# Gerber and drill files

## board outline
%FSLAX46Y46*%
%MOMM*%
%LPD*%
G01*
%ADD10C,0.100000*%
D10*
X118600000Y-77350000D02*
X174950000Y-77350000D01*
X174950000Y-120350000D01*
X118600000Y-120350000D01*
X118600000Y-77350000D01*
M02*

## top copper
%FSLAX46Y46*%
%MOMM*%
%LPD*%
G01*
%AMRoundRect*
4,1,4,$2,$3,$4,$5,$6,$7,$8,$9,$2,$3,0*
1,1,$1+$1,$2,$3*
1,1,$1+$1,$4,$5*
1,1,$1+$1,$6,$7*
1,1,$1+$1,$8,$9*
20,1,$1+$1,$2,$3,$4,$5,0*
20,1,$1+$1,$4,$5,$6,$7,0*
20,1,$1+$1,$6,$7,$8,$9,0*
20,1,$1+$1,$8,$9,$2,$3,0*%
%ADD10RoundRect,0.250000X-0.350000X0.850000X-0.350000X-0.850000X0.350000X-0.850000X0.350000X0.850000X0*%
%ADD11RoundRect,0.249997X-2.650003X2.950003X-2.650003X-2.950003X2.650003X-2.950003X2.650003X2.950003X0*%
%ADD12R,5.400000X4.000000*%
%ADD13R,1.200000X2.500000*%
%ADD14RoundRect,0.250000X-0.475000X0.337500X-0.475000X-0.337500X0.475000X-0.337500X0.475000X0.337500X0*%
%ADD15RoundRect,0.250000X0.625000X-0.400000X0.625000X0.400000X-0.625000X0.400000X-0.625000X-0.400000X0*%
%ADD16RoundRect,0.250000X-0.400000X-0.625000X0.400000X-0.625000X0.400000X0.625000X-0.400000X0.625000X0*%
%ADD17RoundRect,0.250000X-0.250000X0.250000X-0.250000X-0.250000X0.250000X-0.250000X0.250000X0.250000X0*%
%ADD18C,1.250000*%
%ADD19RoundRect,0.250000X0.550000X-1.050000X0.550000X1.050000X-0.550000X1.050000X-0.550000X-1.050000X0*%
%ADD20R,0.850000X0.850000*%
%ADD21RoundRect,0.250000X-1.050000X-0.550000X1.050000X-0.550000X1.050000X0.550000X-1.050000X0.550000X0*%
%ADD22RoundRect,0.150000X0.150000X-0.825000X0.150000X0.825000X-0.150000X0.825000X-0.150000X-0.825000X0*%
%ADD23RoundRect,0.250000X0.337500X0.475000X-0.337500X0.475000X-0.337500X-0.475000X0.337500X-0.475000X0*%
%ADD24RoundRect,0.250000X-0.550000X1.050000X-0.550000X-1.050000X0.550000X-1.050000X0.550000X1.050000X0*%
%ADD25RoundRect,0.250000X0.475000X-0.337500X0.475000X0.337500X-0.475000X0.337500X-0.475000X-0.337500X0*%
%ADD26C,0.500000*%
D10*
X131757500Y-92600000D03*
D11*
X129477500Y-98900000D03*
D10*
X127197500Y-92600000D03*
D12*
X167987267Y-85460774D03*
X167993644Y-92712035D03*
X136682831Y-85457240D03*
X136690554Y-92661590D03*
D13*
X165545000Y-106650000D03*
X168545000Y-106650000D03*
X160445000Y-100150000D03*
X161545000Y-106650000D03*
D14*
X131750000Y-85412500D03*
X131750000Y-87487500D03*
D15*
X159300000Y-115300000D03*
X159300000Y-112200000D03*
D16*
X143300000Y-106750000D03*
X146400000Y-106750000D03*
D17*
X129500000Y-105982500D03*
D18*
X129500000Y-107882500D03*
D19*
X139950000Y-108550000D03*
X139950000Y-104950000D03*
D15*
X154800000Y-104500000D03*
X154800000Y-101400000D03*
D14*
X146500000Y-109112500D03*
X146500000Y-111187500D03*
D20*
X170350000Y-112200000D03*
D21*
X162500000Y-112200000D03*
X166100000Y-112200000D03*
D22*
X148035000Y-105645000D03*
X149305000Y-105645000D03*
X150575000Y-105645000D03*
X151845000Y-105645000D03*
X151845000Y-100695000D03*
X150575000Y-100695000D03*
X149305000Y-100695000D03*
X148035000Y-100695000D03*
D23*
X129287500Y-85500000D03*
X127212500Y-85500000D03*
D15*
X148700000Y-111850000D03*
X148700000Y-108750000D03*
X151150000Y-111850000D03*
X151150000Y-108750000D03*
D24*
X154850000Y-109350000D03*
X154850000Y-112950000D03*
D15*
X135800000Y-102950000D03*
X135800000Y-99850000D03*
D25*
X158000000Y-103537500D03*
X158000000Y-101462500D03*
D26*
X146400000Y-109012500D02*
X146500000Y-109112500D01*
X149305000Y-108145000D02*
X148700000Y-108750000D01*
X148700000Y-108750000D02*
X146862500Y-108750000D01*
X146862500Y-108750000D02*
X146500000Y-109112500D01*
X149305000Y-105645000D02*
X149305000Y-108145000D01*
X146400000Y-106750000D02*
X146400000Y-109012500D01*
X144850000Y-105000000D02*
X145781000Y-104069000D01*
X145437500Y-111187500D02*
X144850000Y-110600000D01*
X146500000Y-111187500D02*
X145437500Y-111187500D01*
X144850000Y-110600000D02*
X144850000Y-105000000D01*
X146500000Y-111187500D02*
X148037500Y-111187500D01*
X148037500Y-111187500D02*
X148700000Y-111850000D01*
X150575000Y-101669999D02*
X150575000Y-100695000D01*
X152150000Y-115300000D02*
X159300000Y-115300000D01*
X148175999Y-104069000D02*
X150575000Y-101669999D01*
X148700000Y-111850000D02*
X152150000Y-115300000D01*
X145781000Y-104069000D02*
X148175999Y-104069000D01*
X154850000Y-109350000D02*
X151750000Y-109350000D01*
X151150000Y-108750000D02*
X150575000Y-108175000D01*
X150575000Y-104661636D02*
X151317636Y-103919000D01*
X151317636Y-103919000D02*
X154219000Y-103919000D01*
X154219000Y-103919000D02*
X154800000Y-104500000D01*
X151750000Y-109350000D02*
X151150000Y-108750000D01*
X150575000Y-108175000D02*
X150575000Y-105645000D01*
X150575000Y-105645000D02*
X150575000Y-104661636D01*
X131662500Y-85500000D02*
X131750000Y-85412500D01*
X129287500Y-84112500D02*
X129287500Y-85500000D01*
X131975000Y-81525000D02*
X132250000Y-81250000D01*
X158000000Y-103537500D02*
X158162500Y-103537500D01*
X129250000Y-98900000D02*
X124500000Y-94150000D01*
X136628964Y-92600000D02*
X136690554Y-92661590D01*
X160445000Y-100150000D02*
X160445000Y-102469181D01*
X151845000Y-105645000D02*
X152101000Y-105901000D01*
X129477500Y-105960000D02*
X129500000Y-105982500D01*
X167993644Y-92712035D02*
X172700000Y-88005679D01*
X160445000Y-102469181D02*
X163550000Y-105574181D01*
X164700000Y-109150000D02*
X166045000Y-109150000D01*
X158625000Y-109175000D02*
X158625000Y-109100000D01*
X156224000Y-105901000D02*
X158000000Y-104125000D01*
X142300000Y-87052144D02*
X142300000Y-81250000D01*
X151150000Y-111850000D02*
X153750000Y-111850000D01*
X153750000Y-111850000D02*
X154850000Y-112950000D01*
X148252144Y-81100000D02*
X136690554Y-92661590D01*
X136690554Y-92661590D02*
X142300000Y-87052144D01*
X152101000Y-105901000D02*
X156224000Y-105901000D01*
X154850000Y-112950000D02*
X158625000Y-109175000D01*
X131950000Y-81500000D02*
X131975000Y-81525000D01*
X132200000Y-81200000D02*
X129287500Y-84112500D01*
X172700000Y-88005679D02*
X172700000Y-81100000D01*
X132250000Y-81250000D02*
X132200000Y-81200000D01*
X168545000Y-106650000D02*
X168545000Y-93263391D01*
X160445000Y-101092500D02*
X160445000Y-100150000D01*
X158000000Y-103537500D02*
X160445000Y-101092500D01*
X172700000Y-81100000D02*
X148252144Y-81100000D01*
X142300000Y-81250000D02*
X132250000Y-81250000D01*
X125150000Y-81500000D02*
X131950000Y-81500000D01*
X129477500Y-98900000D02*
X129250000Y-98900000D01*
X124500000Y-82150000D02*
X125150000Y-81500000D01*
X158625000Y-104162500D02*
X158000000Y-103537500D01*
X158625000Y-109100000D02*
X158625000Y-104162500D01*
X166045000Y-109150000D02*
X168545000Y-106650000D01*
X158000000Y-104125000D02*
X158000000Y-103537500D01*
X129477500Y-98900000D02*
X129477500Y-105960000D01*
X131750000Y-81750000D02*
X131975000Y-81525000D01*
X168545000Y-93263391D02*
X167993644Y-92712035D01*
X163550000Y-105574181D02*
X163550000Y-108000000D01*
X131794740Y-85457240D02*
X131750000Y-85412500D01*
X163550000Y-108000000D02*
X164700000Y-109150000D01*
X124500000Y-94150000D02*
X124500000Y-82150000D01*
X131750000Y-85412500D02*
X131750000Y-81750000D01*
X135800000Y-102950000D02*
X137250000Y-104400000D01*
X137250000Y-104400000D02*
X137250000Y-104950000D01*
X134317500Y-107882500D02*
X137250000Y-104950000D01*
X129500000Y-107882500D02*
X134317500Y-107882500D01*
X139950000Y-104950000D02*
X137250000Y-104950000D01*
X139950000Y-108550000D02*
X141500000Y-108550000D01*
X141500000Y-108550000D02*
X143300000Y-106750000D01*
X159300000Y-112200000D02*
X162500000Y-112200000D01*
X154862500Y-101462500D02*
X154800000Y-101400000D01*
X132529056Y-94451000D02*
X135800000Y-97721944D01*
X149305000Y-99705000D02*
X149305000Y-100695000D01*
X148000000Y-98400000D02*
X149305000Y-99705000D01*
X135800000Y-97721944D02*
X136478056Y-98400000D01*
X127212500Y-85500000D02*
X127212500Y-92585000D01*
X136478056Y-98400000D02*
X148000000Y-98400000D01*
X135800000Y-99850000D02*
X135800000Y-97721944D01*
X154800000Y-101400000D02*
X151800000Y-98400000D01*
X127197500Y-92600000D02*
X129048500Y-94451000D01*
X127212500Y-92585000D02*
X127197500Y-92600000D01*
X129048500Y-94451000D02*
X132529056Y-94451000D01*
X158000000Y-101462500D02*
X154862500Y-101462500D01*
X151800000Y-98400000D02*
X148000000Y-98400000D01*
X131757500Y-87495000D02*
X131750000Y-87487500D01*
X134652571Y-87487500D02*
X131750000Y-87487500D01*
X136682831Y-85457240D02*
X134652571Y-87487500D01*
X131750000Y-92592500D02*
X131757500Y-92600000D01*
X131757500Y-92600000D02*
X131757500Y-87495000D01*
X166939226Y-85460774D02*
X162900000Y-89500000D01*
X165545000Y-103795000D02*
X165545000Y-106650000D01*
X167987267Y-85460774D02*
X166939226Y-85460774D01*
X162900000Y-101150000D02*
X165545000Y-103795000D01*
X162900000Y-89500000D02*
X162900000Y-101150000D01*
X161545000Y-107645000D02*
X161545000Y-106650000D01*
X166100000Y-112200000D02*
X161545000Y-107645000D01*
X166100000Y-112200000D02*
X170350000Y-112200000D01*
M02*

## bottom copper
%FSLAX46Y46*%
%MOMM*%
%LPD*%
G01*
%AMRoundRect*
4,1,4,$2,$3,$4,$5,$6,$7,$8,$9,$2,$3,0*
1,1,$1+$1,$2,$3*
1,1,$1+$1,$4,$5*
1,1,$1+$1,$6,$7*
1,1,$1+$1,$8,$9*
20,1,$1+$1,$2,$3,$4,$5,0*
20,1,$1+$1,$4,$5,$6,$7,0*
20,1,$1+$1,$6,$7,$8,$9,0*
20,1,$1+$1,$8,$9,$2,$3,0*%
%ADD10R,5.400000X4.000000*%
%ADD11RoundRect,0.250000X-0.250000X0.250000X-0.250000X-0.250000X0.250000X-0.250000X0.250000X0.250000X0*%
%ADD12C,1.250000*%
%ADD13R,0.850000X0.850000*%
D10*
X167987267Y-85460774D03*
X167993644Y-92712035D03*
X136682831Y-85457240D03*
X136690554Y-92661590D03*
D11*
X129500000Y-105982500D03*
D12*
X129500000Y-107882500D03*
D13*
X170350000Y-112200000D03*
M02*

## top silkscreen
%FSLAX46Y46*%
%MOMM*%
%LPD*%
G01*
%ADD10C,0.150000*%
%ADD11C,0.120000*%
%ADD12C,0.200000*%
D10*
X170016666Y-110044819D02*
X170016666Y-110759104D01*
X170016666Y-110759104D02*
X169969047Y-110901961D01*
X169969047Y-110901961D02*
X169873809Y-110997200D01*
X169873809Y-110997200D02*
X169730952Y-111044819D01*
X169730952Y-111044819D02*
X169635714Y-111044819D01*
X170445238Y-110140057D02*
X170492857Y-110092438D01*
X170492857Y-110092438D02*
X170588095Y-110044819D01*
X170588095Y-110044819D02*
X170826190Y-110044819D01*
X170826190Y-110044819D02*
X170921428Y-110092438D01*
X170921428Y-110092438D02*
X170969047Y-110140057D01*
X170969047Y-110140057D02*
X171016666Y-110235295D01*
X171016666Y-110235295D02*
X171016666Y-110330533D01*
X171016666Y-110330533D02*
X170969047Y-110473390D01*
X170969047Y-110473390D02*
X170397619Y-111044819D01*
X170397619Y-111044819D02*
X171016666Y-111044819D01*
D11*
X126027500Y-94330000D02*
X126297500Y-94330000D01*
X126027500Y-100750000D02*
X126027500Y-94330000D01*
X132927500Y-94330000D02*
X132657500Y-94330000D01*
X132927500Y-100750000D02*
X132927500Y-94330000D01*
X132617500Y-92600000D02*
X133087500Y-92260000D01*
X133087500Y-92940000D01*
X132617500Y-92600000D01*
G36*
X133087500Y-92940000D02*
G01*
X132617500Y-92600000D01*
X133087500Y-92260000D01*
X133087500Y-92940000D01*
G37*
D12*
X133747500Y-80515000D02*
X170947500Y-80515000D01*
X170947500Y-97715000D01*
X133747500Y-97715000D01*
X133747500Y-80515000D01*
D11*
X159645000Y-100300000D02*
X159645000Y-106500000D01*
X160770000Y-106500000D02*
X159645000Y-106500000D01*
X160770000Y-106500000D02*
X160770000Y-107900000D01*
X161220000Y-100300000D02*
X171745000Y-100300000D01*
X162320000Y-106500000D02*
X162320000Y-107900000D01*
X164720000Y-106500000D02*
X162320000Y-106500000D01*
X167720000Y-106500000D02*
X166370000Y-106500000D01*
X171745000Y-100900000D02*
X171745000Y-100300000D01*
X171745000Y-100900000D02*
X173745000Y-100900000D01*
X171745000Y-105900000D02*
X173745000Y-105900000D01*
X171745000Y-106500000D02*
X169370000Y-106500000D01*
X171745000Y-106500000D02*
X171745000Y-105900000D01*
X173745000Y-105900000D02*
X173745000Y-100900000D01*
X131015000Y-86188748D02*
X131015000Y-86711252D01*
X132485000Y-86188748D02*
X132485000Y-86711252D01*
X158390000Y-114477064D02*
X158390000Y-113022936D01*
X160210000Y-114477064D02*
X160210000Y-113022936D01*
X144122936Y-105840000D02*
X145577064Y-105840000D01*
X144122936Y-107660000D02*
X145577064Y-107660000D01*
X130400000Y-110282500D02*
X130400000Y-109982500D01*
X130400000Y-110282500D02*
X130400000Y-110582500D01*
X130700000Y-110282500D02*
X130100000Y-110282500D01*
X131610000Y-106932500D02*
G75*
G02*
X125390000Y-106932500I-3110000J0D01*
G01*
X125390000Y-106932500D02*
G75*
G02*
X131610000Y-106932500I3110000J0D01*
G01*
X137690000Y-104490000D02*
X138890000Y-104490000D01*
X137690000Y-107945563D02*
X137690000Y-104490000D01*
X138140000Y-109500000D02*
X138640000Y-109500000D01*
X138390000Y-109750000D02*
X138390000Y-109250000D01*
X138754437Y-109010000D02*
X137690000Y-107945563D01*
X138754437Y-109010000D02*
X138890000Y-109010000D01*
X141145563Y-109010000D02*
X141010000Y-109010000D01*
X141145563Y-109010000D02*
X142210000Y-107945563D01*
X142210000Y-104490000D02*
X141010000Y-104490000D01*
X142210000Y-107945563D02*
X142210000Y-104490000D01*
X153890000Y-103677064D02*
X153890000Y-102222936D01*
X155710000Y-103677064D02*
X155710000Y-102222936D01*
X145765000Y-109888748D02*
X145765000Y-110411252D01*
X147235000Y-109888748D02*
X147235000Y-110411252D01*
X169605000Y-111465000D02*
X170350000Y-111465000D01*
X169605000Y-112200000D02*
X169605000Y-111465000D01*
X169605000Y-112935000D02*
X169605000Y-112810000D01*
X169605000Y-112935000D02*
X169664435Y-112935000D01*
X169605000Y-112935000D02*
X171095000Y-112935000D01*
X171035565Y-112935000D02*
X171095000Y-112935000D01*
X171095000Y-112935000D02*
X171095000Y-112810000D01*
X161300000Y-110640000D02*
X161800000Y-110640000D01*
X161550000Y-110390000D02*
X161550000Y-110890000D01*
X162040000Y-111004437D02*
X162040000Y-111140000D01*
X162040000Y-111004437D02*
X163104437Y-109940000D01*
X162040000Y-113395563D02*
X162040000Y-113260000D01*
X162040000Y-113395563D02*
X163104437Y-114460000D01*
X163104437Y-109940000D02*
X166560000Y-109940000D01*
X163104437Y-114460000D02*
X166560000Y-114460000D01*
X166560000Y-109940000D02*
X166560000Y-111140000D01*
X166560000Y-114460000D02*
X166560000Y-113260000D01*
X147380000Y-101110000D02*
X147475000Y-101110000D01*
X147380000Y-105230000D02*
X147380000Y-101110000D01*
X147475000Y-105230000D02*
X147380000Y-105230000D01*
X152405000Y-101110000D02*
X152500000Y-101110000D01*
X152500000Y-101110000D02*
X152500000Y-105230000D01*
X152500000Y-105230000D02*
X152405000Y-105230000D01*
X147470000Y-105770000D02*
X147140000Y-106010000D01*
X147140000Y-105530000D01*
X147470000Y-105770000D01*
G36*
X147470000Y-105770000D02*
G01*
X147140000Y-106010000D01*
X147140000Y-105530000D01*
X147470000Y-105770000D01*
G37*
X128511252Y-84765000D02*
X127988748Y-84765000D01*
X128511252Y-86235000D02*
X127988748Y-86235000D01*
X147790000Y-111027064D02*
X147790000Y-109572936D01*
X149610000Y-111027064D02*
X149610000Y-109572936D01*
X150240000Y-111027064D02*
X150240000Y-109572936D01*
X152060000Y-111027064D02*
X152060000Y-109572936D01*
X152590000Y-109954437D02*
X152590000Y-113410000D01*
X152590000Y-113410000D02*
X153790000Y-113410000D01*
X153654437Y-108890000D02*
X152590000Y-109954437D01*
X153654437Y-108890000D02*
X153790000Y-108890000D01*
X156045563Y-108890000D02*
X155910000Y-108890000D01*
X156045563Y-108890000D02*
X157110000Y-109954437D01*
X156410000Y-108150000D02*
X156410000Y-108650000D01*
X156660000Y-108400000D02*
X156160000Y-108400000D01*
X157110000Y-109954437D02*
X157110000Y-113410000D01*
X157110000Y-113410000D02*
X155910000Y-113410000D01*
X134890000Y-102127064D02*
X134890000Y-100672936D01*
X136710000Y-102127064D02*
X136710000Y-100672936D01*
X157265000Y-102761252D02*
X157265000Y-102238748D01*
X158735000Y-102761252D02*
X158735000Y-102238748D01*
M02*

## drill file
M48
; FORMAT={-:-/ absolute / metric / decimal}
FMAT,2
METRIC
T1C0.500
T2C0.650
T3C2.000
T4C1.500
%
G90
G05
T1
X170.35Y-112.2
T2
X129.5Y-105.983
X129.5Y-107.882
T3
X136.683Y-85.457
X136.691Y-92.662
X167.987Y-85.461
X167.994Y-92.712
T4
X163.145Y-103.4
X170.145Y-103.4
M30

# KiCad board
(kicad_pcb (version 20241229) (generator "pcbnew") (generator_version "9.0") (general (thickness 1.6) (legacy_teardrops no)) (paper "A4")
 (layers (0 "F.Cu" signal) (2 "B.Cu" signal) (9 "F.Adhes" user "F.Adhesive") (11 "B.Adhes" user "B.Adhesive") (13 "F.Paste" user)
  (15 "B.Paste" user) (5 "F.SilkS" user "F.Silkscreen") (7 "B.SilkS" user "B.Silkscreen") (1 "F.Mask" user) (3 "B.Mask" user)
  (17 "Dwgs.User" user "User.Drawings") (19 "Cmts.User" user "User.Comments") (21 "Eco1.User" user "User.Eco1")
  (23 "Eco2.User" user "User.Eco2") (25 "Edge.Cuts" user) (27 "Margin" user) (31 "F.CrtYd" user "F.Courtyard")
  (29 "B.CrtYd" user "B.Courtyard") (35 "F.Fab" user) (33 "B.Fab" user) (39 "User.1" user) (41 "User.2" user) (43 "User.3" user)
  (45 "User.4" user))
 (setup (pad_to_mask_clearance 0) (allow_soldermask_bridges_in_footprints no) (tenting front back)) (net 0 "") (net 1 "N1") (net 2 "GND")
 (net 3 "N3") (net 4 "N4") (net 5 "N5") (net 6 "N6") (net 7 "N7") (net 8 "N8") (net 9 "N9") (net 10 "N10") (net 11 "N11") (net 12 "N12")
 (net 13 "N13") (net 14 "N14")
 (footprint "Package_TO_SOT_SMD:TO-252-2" (layer "F.Cu") (at 129.4775 97.64 -90)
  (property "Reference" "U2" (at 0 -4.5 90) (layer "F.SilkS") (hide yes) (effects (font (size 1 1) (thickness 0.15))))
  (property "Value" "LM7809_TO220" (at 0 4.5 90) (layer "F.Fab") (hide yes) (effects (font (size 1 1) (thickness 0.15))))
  (fp_line (start -3.31 3.45) (end -3.31 3.18) (stroke (width 0.12) (type solid)) (layer "F.SilkS"))
  (fp_line (start 3.11 3.45) (end -3.31 3.45) (stroke (width 0.12) (type solid)) (layer "F.SilkS"))
  (fp_line (start -3.31 -3.45) (end -3.31 -3.18) (stroke (width 0.12) (type solid)) (layer "F.SilkS"))
  (fp_line (start 3.11 -3.45) (end -3.31 -3.45) (stroke (width 0.12) (type solid)) (layer "F.SilkS"))
  (fp_poly (pts (xy -5.04 -3.14) (xy -5.38 -3.61) (xy -4.7 -3.61)) (stroke (width 0.12) (type solid)) (fill yes) (layer "F.SilkS"))
  (pad "" smd roundrect (at -0.415 -1.525 270) (size 3.05 2.75) (layers "F.Paste") (roundrect_rratio 0.090909))
  (pad "" smd roundrect (at -0.415 1.525 270) (size 3.05 2.75) (layers "F.Paste") (roundrect_rratio 0.090909))
  (pad "" smd roundrect (at 2.935 -1.525 270) (size 3.05 2.75) (layers "F.Paste") (roundrect_rratio 0.090909))
  (pad "" smd roundrect (at 2.935 1.525 270) (size 3.05 2.75) (layers "F.Paste") (roundrect_rratio 0.090909))
  (pad "1" smd roundrect (at -5.04 -2.28 270) (size 2.2 1.2) (layers "F.Cu" "F.Mask" "F.Paste") (roundrect_rratio 0.208333) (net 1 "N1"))
  (pad "2" smd roundrect (at 1.26 0 270) (size 6.4 5.8) (layers "F.Cu" "F.Mask") (roundrect_rratio 0.043103) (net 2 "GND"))
  (pad "3" smd roundrect (at -5.04 2.28 270) (size 2.2 1.2) (layers "F.Cu" "F.Mask" "F.Paste") (roundrect_rratio 0.208333) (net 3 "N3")))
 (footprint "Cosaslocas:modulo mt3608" (layer "F.Cu") (at 133.7475 97.715)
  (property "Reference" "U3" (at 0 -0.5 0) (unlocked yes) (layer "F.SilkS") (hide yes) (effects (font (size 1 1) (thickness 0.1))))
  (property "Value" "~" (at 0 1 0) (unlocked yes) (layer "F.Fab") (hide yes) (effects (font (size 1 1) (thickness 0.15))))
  (fp_rect (start 0 -17.2) (end 37.2 0) (stroke (width 0.2) (type solid)) (fill no) (layer "F.SilkS"))
  (pad "1" thru_hole rect (at 34.239767 -12.254226) (size 5.4 4) (drill 2) (layers "*.Cu" "*.Mask") (remove_unused_layers no) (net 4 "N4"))
  (pad "2" thru_hole rect (at 34.246144 -5.002965) (size 5.4 4) (drill 2) (layers "*.Cu" "*.Mask") (remove_unused_layers no) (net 2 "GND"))
  (pad "3" thru_hole rect (at 2.935331 -12.25776) (size 5.4 4) (drill 2) (layers "*.Cu" "*.Mask") (remove_unused_layers no) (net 1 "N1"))
  (pad "4" thru_hole rect (at 2.943054 -5.05341) (size 5.4 4) (drill 2) (layers "*.Cu" "*.Mask") (remove_unused_layers no) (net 2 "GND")))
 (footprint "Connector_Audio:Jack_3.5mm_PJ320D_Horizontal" (layer "F.Cu") (at 165.37 103.4 180)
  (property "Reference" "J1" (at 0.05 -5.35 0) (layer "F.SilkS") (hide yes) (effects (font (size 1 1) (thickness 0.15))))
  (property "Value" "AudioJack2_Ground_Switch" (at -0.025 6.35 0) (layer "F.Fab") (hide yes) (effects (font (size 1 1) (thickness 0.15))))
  (fp_line (start 5.725 3.1) (end 5.725 -3.1) (stroke (width 0.12) (type solid)) (layer "F.SilkS"))
  (fp_line (start 4.6 -3.1) (end 5.725 -3.1) (stroke (width 0.12) (type solid)) (layer "F.SilkS"))
  (fp_line (start 4.6 -3.1) (end 4.6 -4.5) (stroke (width 0.12) (type solid)) (layer "F.SilkS"))
  (fp_line (start 4.15 3.1) (end -6.375 3.1) (stroke (width 0.12) (type solid)) (layer "F.SilkS"))
  (fp_line (start 3.05 -3.1) (end 3.05 -4.5) (stroke (width 0.12) (type solid)) (layer "F.SilkS"))
  (fp_line (start 0.65 -3.1) (end 3.05 -3.1) (stroke (width 0.12) (type solid)) (layer "F.SilkS"))
  (fp_line (start -2.35 -3.1) (end -1 -3.1) (stroke (width 0.12) (type solid)) (layer "F.SilkS"))
  (fp_line (start -6.375 2.5) (end -6.375 3.1) (stroke (width 0.12) (type solid)) (layer "F.SilkS"))
  (fp_line (start -6.375 2.5) (end -8.375 2.5) (stroke (width 0.12) (type solid)) (layer "F.SilkS"))
  (fp_line (start -6.375 -2.5) (end -8.375 -2.5) (stroke (width 0.12) (type solid)) (layer "F.SilkS"))
  (fp_line (start -6.375 -3.1) (end -4 -3.1) (stroke (width 0.12) (type solid)) (layer "F.SilkS"))
  (fp_line (start -6.375 -3.1) (end -6.375 -2.5) (stroke (width 0.12) (type solid)) (layer "F.SilkS"))
  (fp_line (start -8.375 -2.5) (end -8.375 2.5) (stroke (width 0.12) (type solid)) (layer "F.SilkS"))
  (pad "" np_thru_hole circle (at -4.775 0 180) (size 1.5 1.5) (drill 1.5) (layers "*.Cu" "*.Mask"))
  (pad "" np_thru_hole circle (at 2.225 0 180) (size 1.5 1.5) (drill 1.5) (layers "*.Cu" "*.Mask"))
  (pad "R1" smd rect (at -0.175 -3.25 180) (size 1.2 2.5) (layers "F.Cu" "F.Mask" "F.Paste") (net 4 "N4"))
  (pad "R2" smd rect (at -3.175 -3.25 180) (size 1.2 2.5) (layers "F.Cu" "F.Mask" "F.Paste") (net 2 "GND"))
  (pad "S" smd rect (at 4.925 3.25 180) (size 1.2 2.5) (layers "F.Cu" "F.Mask" "F.Paste") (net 2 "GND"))
  (pad "T" smd rect (at 3.825 -3.25 180) (size 1.2 2.5) (layers "F.Cu" "F.Mask" "F.Paste") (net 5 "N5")))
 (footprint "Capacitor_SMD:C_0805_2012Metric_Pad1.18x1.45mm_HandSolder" (layer "F.Cu") (at 131.75 86.45 -90)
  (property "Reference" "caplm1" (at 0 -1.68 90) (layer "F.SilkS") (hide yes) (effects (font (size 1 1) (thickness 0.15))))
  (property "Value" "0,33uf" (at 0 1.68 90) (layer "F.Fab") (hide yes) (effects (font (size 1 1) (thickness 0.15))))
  (fp_line (start -0.261252 0.735) (end 0.261252 0.735) (stroke (width 0.12) (type solid)) (layer "F.SilkS"))
  (fp_line (start -0.261252 -0.735) (end 0.261252 -0.735) (stroke (width 0.12) (type solid)) (layer "F.SilkS"))
  (pad "1" smd roundrect (at -1.0375 0 270) (size 1.175 1.45) (layers "F.Cu" "F.Mask" "F.Paste") (roundrect_rratio 0.212766) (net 2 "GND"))
  (pad "2" smd roundrect (at 1.0375 0 270) (size 1.175 1.45) (layers "F.Cu" "F.Mask" "F.Paste") (roundrect_rratio 0.212766) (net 1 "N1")))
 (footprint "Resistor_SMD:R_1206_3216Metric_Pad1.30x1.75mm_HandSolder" (layer "F.Cu") (at 159.3 113.75 90)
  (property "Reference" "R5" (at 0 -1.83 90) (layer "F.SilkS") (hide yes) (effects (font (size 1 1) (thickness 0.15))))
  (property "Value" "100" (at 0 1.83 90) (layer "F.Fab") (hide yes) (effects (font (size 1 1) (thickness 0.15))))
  (fp_line (start -0.727064 -0.91) (end 0.727064 -0.91) (stroke (width 0.12) (type solid)) (layer "F.SilkS"))
  (fp_line (start -0.727064 0.91) (end 0.727064 0.91) (stroke (width 0.12) (type solid)) (layer "F.SilkS"))
  (pad "1" smd roundrect (at -1.55 0 90) (size 1.3 1.75) (layers "F.Cu" "F.Mask" "F.Paste") (roundrect_rratio 0.192308) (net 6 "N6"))
  (pad "2" smd roundrect (at 1.55 0 90) (size 1.3 1.75) (layers "F.Cu" "F.Mask" "F.Paste") (roundrect_rratio 0.192308) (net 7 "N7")))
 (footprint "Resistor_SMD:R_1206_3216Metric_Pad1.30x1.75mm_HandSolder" (layer "F.Cu") (at 144.85 106.75)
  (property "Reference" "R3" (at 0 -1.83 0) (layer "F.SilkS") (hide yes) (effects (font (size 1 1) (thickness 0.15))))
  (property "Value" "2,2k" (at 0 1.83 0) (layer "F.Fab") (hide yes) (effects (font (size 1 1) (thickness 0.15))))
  (fp_line (start -0.727064 -0.91) (end 0.727064 -0.91) (stroke (width 0.12) (type solid)) (layer "F.SilkS"))
  (fp_line (start -0.727064 0.91) (end 0.727064 0.91) (stroke (width 0.12) (type solid)) (layer "F.SilkS"))
  (pad "1" smd roundrect (at -1.55 0) (size 1.3 1.75) (layers "F.Cu" "F.Mask" "F.Paste") (roundrect_rratio 0.192308) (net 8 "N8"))
  (pad "2" smd roundrect (at 1.55 0) (size 1.3 1.75) (layers "F.Cu" "F.Mask" "F.Paste") (roundrect_rratio 0.192308) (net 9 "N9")))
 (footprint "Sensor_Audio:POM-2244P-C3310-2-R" (layer "F.Cu") (at 129.5 105.9825 -90)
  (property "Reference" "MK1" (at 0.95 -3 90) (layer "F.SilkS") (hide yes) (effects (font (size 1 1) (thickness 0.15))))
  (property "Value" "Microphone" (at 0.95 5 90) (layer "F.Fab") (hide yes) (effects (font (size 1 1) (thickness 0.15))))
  (fp_line (start 4.3 -0.9) (end 4 -0.9) (stroke (width 0.12) (type default)) (layer "F.SilkS"))
  (fp_line (start 4.3 -0.9) (end 4.6 -0.9) (stroke (width 0.12) (type default)) (layer "F.SilkS"))
  (fp_line (start 4.3 -1.2) (end 4.3 -0.6) (stroke (width 0.12) (type default)) (layer "F.SilkS"))
  (fp_circle (center 0.95 1) (end 4.06 1) (stroke (width 0.12) (type default)) (fill no) (layer "F.SilkS"))
  (pad "1" thru_hole roundrect (at 0 0 270) (size 1 1) (drill 0.65) (layers "*.Cu" "*.Mask") (remove_unused_layers no)
   (roundrect_rratio 0.25) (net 2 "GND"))
  (pad "2" thru_hole circle (at 1.9 0 270) (size 1.25 1.25) (drill 0.65) (layers "*.Cu" "*.Mask") (remove_unused_layers no) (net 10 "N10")))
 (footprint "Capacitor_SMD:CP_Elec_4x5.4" (layer "F.Cu") (at 139.95 106.75 90)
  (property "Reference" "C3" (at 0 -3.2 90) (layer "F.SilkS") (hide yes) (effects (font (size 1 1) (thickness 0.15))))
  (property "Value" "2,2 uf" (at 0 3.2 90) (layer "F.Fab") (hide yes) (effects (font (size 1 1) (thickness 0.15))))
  (fp_line (start 2.26 -2.26) (end 2.26 -1.06) (stroke (width 0.12) (type solid)) (layer "F.SilkS"))
  (fp_line (start -1.195563 -2.26) (end 2.26 -2.26) (stroke (width 0.12) (type solid)) (layer "F.SilkS"))
  (fp_line (start -2.75 -1.81) (end -2.75 -1.31) (stroke (width 0.12) (type solid)) (layer "F.SilkS"))
  (fp_line (start -3 -1.56) (end -2.5 -1.56) (stroke (width 0.12) (type solid)) (layer "F.SilkS"))
  (fp_line (start -2.26 -1.195563) (end -1.195563 -2.26) (stroke (width 0.12) (type solid)) (layer "F.SilkS"))
  (fp_line (start -2.26 -1.195563) (end -2.26 -1.06) (stroke (width 0.12) (type solid)) (layer "F.SilkS"))
  (fp_line (start -2.26 1.195563) (end -2.26 1.06) (stroke (width 0.12) (type solid)) (layer "F.SilkS"))
  (fp_line (start -2.26 1.195563) (end -1.195563 2.26) (stroke (width 0.12) (type solid)) (layer "F.SilkS"))
  (fp_line (start 2.26 2.26) (end 2.26 1.06) (stroke (width 0.12) (type solid)) (layer "F.SilkS"))
  (fp_line (start -1.195563 2.26) (end 2.26 2.26) (stroke (width 0.12) (type solid)) (layer "F.SilkS"))
  (pad "1" smd roundrect (at -1.8 0 90) (size 2.6 1.6) (layers "F.Cu" "F.Mask" "F.Paste") (roundrect_rratio 0.15625) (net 8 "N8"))
  (pad "2" smd roundrect (at 1.8 0 90) (size 2.6 1.6) (layers "F.Cu" "F.Mask" "F.Paste") (roundrect_rratio 0.15625) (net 10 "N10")))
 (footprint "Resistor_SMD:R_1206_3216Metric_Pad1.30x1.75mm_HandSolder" (layer "F.Cu") (at 154.8 102.95 90)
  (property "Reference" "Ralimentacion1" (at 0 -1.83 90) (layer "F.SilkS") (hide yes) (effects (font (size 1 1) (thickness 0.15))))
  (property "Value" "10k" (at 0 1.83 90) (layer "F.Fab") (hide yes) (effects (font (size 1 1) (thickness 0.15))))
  (fp_line (start -0.727064 -0.91) (end 0.727064 -0.91) (stroke (width 0.12) (type solid)) (layer "F.SilkS"))
  (fp_line (start -0.727064 0.91) (end 0.727064 0.91) (stroke (width 0.12) (type solid)) (layer "F.SilkS"))
  (pad "1" smd roundrect (at -1.55 0 90) (size 1.3 1.75) (layers "F.Cu" "F.Mask" "F.Paste") (roundrect_rratio 0.192308) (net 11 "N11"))
  (pad "2" smd roundrect (at 1.55 0 90) (size 1.3 1.75) (layers "F.Cu" "F.Mask" "F.Paste") (roundrect_rratio 0.192308) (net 3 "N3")))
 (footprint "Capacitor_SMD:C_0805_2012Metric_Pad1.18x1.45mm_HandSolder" (layer "F.Cu") (at 146.5 110.15 -90)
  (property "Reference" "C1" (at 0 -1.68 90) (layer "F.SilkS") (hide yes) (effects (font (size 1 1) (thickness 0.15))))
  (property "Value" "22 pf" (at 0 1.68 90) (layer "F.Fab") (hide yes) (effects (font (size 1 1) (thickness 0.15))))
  (fp_line (start -0.261252 0.735) (end 0.261252 0.735) (stroke (width 0.12) (type solid)) (layer "F.SilkS"))
  (fp_line (start -0.261252 -0.735) (end 0.261252 -0.735) (stroke (width 0.12) (type solid)) (layer "F.SilkS"))
  (pad "1" smd roundrect (at -1.0375 0 270) (size 1.175 1.45) (layers "F.Cu" "F.Mask" "F.Paste") (roundrect_rratio 0.212766) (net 9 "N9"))
  (pad "2" smd roundrect (at 1.0375 0 270) (size 1.175 1.45) (layers "F.Cu" "F.Mask" "F.Paste") (roundrect_rratio 0.212766) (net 6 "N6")))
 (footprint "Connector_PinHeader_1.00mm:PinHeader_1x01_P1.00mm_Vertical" (layer "F.Cu") (at 170.35 112.2)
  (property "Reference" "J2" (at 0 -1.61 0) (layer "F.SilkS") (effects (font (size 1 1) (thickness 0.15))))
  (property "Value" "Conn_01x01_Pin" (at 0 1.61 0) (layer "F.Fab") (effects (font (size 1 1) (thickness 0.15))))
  (fp_line (start -0.745 -0.735) (end 0 -0.735) (stroke (width 0.12) (type solid)) (layer "F.SilkS"))
  (fp_line (start -0.745 0) (end -0.745 -0.735) (stroke (width 0.12) (type solid)) (layer "F.SilkS"))
  (fp_line (start -0.745 0.735) (end -0.745 0.61) (stroke (width 0.12) (type solid)) (layer "F.SilkS"))
  (fp_line (start -0.745 0.735) (end -0.685565 0.735) (stroke (width 0.12) (type solid)) (layer "F.SilkS"))
  (fp_line (start -0.745 0.735) (end 0.745 0.735) (stroke (width 0.12) (type solid)) (layer "F.SilkS"))
  (fp_line (start 0.685565 0.735) (end 0.745 0.735) (stroke (width 0.12) (type solid)) (layer "F.SilkS"))
  (fp_line (start 0.745 0.735) (end 0.745 0.61) (stroke (width 0.12) (type solid)) (layer "F.SilkS"))
  (pad "1" thru_hole rect (at 0 0) (size 0.85 0.85) (drill 0.5) (layers "*.Cu" "*.Mask") (remove_unused_layers no) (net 5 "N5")))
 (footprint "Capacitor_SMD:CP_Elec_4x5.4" (layer "F.Cu") (at 164.3 112.2)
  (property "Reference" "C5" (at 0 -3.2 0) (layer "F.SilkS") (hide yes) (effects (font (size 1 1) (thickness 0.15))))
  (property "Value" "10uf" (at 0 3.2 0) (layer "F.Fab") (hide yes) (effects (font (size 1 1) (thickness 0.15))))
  (fp_line (start -3 -1.56) (end -2.5 -1.56) (stroke (width 0.12) (type solid)) (layer "F.SilkS"))
  (fp_line (start -2.75 -1.81) (end -2.75 -1.31) (stroke (width 0.12) (type solid)) (layer "F.SilkS"))
  (fp_line (start -2.26 -1.195563) (end -2.26 -1.06) (stroke (width 0.12) (type solid)) (layer "F.SilkS"))
  (fp_line (start -2.26 -1.195563) (end -1.195563 -2.26) (stroke (width 0.12) (type solid)) (layer "F.SilkS"))
  (fp_line (start -2.26 1.195563) (end -2.26 1.06) (stroke (width 0.12) (type solid)) (layer "F.SilkS"))
  (fp_line (start -2.26 1.195563) (end -1.195563 2.26) (stroke (width 0.12) (type solid)) (layer "F.SilkS"))
  (fp_line (start -1.195563 -2.26) (end 2.26 -2.26) (stroke (width 0.12) (type solid)) (layer "F.SilkS"))
  (fp_line (start -1.195563 2.26) (end 2.26 2.26) (stroke (width 0.12) (type solid)) (layer "F.SilkS"))
  (fp_line (start 2.26 -2.26) (end 2.26 -1.06) (stroke (width 0.12) (type solid)) (layer "F.SilkS"))
  (fp_line (start 2.26 2.26) (end 2.26 1.06) (stroke (width 0.12) (type solid)) (layer "F.SilkS"))
  (pad "1" smd roundrect (at -1.8 0) (size 2.6 1.6) (layers "F.Cu" "F.Mask" "F.Paste") (roundrect_rratio 0.15625) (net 7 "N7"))
  (pad "2" smd roundrect (at 1.8 0) (size 2.6 1.6) (layers "F.Cu" "F.Mask" "F.Paste") (roundrect_rratio 0.15625) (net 5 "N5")))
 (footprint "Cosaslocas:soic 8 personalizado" (layer "F.Cu") (at 149.95 103.12 90)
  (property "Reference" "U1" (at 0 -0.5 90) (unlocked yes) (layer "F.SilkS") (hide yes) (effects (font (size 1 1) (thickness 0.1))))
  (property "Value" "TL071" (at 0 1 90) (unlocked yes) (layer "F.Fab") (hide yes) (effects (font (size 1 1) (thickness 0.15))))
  (fp_line (start 2.01 -2.57) (end 2.01 -2.475) (stroke (width 0.12) (type solid)) (layer "F.SilkS"))
  (fp_line (start -2.11 -2.57) (end 2.01 -2.57) (stroke (width 0.12) (type solid)) (layer "F.SilkS"))
  (fp_line (start -2.11 -2.475) (end -2.11 -2.57) (stroke (width 0.12) (type solid)) (layer "F.SilkS"))
  (fp_line (start 2.01 2.455) (end 2.01 2.55) (stroke (width 0.12) (type solid)) (layer "F.SilkS"))
  (fp_line (start 2.01 2.55) (end -2.11 2.55) (stroke (width 0.12) (type solid)) (layer "F.SilkS"))
  (fp_line (start -2.11 2.55) (end -2.11 2.455) (stroke (width 0.12) (type solid)) (layer "F.SilkS"))
  (fp_poly (pts (xy -2.65 -2.48) (xy -2.89 -2.81) (xy -2.41 -2.81)) (stroke (width 0.12) (type solid)) (fill yes) (layer "F.SilkS"))
  (pad "1" smd roundrect (at -2.525 -1.915 90) (size 1.95 0.6) (layers "F.Cu" "F.Mask" "F.Paste") (roundrect_rratio 0.25) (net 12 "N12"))
  (pad "2" smd roundrect (at -2.525 -0.645 90) (size 1.95 0.6) (layers "F.Cu" "F.Mask" "F.Paste") (roundrect_rratio 0.25) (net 9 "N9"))
  (pad "3" smd roundrect (at -2.525 0.625 90) (size 1.95 0.6) (layers "F.Cu" "F.Mask" "F.Paste") (roundrect_rratio 0.25) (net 11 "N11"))
  (pad "4" smd roundrect (at -2.525 1.895 90) (size 1.95 0.6) (layers "F.Cu" "F.Mask" "F.Paste") (roundrect_rratio 0.25) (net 2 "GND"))
  (pad "5" smd roundrect (at 2.425 1.895 90) (size 1.95 0.6) (layers "F.Cu" "F.Mask" "F.Paste") (roundrect_rratio 0.25) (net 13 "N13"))
  (pad "6" smd roundrect (at 2.425 0.625 90) (size 1.95 0.6) (layers "F.Cu" "F.Mask" "F.Paste") (roundrect_rratio 0.25) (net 6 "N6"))
  (pad "7" smd roundrect (at 2.425 -0.645 90) (size 1.95 0.6) (layers "F.Cu" "F.Mask" "F.Paste") (roundrect_rratio 0.25) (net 3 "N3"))
  (pad "8" smd roundrect (at 2.425 -1.915 90) (size 1.95 0.6) (layers "F.Cu" "F.Mask" "F.Paste") (roundrect_rratio 0.25) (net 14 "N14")))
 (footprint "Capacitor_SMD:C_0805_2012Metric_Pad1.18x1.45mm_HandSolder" (layer "F.Cu") (at 128.25 85.5 180)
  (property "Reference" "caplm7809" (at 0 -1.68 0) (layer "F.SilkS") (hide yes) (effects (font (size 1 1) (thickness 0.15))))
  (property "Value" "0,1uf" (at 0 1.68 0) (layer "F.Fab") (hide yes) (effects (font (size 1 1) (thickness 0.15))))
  (fp_line (start -0.261252 0.735) (end 0.261252 0.735) (stroke (width 0.12) (type solid)) (layer "F.SilkS"))
  (fp_line (start -0.261252 -0.735) (end 0.261252 -0.735) (stroke (width 0.12) (type solid)) (layer "F.SilkS"))
  (pad "1" smd roundrect (at -1.0375 0 180) (size 1.175 1.45) (layers "F.Cu" "F.Mask" "F.Paste") (roundrect_rratio 0.212766) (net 2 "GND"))
  (pad "2" smd roundrect (at 1.0375 0 180) (size 1.175 1.45) (layers "F.Cu" "F.Mask" "F.Paste") (roundrect_rratio 0.212766) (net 3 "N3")))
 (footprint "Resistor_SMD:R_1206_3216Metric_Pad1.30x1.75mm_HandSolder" (layer "F.Cu") (at 148.7 110.3 90)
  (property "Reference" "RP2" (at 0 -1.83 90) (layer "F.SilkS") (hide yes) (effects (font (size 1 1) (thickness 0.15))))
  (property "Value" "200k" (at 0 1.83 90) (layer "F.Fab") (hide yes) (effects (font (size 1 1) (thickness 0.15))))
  (fp_line (start -0.727064 -0.91) (end 0.727064 -0.91) (stroke (width 0.12) (type solid)) (layer "F.SilkS"))
  (fp_line (start -0.727064 0.91) (end 0.727064 0.91) (stroke (width 0.12) (type solid)) (layer "F.SilkS"))
  (pad "1" smd roundrect (at -1.55 0 90) (size 1.3 1.75) (layers "F.Cu" "F.Mask" "F.Paste") (roundrect_rratio 0.192308) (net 6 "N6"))
  (pad "2" smd roundrect (at 1.55 0 90) (size 1.3 1.75) (layers "F.Cu" "F.Mask" "F.Paste") (roundrect_rratio 0.192308) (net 9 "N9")))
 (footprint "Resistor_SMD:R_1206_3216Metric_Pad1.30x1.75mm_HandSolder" (layer "F.Cu") (at 151.15 110.3 90)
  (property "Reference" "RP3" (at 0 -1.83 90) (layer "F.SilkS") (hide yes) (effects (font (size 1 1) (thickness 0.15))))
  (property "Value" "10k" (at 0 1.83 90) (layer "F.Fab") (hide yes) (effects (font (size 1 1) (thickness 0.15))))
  (fp_line (start -0.727064 -0.91) (end 0.727064 -0.91) (stroke (width 0.12) (type solid)) (layer "F.SilkS"))
  (fp_line (start -0.727064 0.91) (end 0.727064 0.91) (stroke (width 0.12) (type solid)) (layer "F.SilkS"))
  (pad "1" smd roundrect (at -1.55 0 90) (size 1.3 1.75) (layers "F.Cu" "F.Mask" "F.Paste") (roundrect_rratio 0.192308) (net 2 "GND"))
  (pad "2" smd roundrect (at 1.55 0 90) (size 1.3 1.75) (layers "F.Cu" "F.Mask" "F.Paste") (roundrect_rratio 0.192308) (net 11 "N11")))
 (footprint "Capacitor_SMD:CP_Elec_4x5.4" (layer "F.Cu") (at 154.85 111.15 -90)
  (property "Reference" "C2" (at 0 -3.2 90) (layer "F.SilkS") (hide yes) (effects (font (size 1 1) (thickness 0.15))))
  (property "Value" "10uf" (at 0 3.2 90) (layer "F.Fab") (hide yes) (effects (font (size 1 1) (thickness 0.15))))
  (fp_line (start -1.195563 2.26) (end 2.26 2.26) (stroke (width 0.12) (type solid)) (layer "F.SilkS"))
  (fp_line (start 2.26 2.26) (end 2.26 1.06) (stroke (width 0.12) (type solid)) (layer "F.SilkS"))
  (fp_line (start -2.26 1.195563) (end -1.195563 2.26) (stroke (width 0.12) (type solid)) (layer "F.SilkS"))
  (fp_line (start -2.26 1.195563) (end -2.26 1.06) (stroke (width 0.12) (type solid)) (layer "F.SilkS"))
  (fp_line (start -2.26 -1.195563) (end -2.26 -1.06) (stroke (width 0.12) (type solid)) (layer "F.SilkS"))
  (fp_line (start -2.26 -1.195563) (end -1.195563 -2.26) (stroke (width 0.12) (type solid)) (layer "F.SilkS"))
  (fp_line (start -3 -1.56) (end -2.5 -1.56) (stroke (width 0.12) (type solid)) (layer "F.SilkS"))
  (fp_line (start -2.75 -1.81) (end -2.75 -1.31) (stroke (width 0.12) (type solid)) (layer "F.SilkS"))
  (fp_line (start -1.195563 -2.26) (end 2.26 -2.26) (stroke (width 0.12) (type solid)) (layer "F.SilkS"))
  (fp_line (start 2.26 -2.26) (end 2.26 -1.06) (stroke (width 0.12) (type solid)) (layer "F.SilkS"))
  (pad "1" smd roundrect (at -1.8 0 270) (size 2.6 1.6) (layers "F.Cu" "F.Mask" "F.Paste") (roundrect_rratio 0.15625) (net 11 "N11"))
  (pad "2" smd roundrect (at 1.8 0 270) (size 2.6 1.6) (layers "F.Cu" "F.Mask" "F.Paste") (roundrect_rratio 0.15625) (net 2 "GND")))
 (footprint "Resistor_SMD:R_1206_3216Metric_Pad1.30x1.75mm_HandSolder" (layer "F.Cu") (at 135.8 101.4 90)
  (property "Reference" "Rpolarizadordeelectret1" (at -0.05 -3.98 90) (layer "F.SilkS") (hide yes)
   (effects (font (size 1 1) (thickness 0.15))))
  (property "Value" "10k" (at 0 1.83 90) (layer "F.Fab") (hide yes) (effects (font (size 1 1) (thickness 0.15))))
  (fp_line (start -0.727064 -0.91) (end 0.727064 -0.91) (stroke (width 0.12) (type solid)) (layer "F.SilkS"))
  (fp_line (start -0.727064 0.91) (end 0.727064 0.91) (stroke (width 0.12) (type solid)) (layer "F.SilkS"))
  (pad "1" smd roundrect (at -1.55 0 90) (size 1.3 1.75) (layers "F.Cu" "F.Mask" "F.Paste") (roundrect_rratio 0.192308) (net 10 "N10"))
  (pad "2" smd roundrect (at 1.55 0 90) (size 1.3 1.75) (layers "F.Cu" "F.Mask" "F.Paste") (roundrect_rratio 0.192308) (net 3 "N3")))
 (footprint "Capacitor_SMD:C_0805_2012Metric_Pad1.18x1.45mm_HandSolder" (layer "F.Cu") (at 158 102.5 90)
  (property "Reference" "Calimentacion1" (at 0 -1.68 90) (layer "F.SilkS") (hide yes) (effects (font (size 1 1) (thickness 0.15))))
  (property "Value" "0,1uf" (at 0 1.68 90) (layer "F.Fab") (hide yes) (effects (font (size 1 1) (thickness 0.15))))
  (fp_line (start -0.261252 -0.735) (end 0.261252 -0.735) (stroke (width 0.12) (type solid)) (layer "F.SilkS"))
  (fp_line (start -0.261252 0.735) (end 0.261252 0.735) (stroke (width 0.12) (type solid)) (layer "F.SilkS"))
  (pad "1" smd roundrect (at -1.0375 0 90) (size 1.175 1.45) (layers "F.Cu" "F.Mask" "F.Paste") (roundrect_rratio 0.212766) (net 2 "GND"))
  (pad "2" smd roundrect (at 1.0375 0 90) (size 1.175 1.45) (layers "F.Cu" "F.Mask" "F.Paste") (roundrect_rratio 0.212766) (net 3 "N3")))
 (gr_rect (start 118.6 77.35) (end 174.95 120.35) (stroke (width 0.1) (type solid)) (fill no) (layer "Edge.Cuts"))
 (segment (start 146.4 109.0125) (end 146.5 109.1125) (width 0.5) (layer "F.Cu") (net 9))
 (segment (start 149.305 108.145) (end 148.7 108.75) (width 0.5) (layer "F.Cu") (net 9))
 (segment (start 148.7 108.75) (end 146.8625 108.75) (width 0.5) (layer "F.Cu") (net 9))
 (segment (start 146.8625 108.75) (end 146.5 109.1125) (width 0.5) (layer "F.Cu") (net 9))
 (segment (start 149.305 105.645) (end 149.305 108.145) (width 0.5) (layer "F.Cu") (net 9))
 (segment (start 146.4 106.75) (end 146.4 109.0125) (width 0.5) (layer "F.Cu") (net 9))
 (segment (start 144.85 105) (end 145.781 104.069) (width 0.5) (layer "F.Cu") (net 6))
 (segment (start 145.4375 111.1875) (end 144.85 110.6) (width 0.5) (layer "F.Cu") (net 6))
 (segment (start 146.5 111.1875) (end 145.4375 111.1875) (width 0.5) (layer "F.Cu") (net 6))
 (segment (start 144.85 110.6) (end 144.85 105) (width 0.5) (layer "F.Cu") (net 6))
 (segment (start 146.5 111.1875) (end 148.0375 111.1875) (width 0.5) (layer "F.Cu") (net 6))
 (segment (start 148.0375 111.1875) (end 148.7 111.85) (width 0.5) (layer "F.Cu") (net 6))
 (segment (start 150.575 101.669999) (end 150.575 100.695) (width 0.5) (layer "F.Cu") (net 6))
 (segment (start 152.15 115.3) (end 159.3 115.3) (width 0.5) (layer "F.Cu") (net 6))
 (segment (start 148.175999 104.069) (end 150.575 101.669999) (width 0.5) (layer "F.Cu") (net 6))
 (segment (start 148.7 111.85) (end 152.15 115.3) (width 0.5) (layer "F.Cu") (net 6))
 (segment (start 145.781 104.069) (end 148.175999 104.069) (width 0.5) (layer "F.Cu") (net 6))
 (segment (start 154.85 109.35) (end 151.75 109.35) (width 0.5) (layer "F.Cu") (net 11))
 (segment (start 151.15 108.75) (end 150.575 108.175) (width 0.5) (layer "F.Cu") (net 11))
 (segment (start 150.575 104.661636) (end 151.317636 103.919) (width 0.5) (layer "F.Cu") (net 11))
 (segment (start 151.317636 103.919) (end 154.219 103.919) (width 0.5) (layer "F.Cu") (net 11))
 (segment (start 154.219 103.919) (end 154.8 104.5) (width 0.5) (layer "F.Cu") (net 11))
 (segment (start 151.75 109.35) (end 151.15 108.75) (width 0.5) (layer "F.Cu") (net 11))
 (segment (start 150.575 108.175) (end 150.575 105.645) (width 0.5) (layer "F.Cu") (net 11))
 (segment (start 150.575 105.645) (end 150.575 104.661636) (width 0.5) (layer "F.Cu") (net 11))
 (segment (start 131.6625 85.5) (end 131.75 85.4125) (width 0.5) (layer "F.Cu") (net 2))
 (segment (start 129.2875 84.1125) (end 129.2875 85.5) (width 0.5) (layer "F.Cu") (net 2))
 (segment (start 131.975 81.525) (end 132.25 81.25) (width 0.5) (layer "F.Cu") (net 2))
 (segment (start 158 103.5375) (end 158.1625 103.5375) (width 0.5) (layer "F.Cu") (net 2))
 (segment (start 129.25 98.9) (end 124.5 94.15) (width 0.5) (layer "F.Cu") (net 2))
 (segment (start 136.628964 92.6) (end 136.690554 92.66159) (width 0.5) (layer "F.Cu") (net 2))
 (segment (start 160.445 100.15) (end 160.445 102.469181) (width 0.5) (layer "F.Cu") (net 2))
 (segment (start 151.845 105.645) (end 152.101 105.901) (width 0.5) (layer "F.Cu") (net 2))
 (segment (start 129.4775 105.96) (end 129.5 105.9825) (width 0.5) (layer "F.Cu") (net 2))
 (segment (start 167.993644 92.712035) (end 172.7 88.005679) (width 0.5) (layer "F.Cu") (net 2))
 (segment (start 160.445 102.469181) (end 163.55 105.574181) (width 0.5) (layer "F.Cu") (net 2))
 (segment (start 164.7 109.15) (end 166.045 109.15) (width 0.5) (layer "F.Cu") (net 2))
 (segment (start 158.625 109.175) (end 158.625 109.1) (width 0.5) (layer "F.Cu") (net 2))
 (segment (start 156.224 105.901) (end 158 104.125) (width 0.5) (layer "F.Cu") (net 2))
 (segment (start 142.3 87.052144) (end 142.3 81.25) (width 0.5) (layer "F.Cu") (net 2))
 (segment (start 151.15 111.85) (end 153.75 111.85) (width 0.5) (layer "F.Cu") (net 2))
 (segment (start 153.75 111.85) (end 154.85 112.95) (width 0.5) (layer "F.Cu") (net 2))
 (segment (start 148.252144 81.1) (end 136.690554 92.66159) (width 0.5) (layer "F.Cu") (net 2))
 (segment (start 136.690554 92.66159) (end 142.3 87.052144) (width 0.5) (layer "F.Cu") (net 2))
 (segment (start 152.101 105.901) (end 156.224 105.901) (width 0.5) (layer "F.Cu") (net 2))
 (segment (start 154.85 112.95) (end 158.625 109.175) (width 0.5) (layer "F.Cu") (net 2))
 (segment (start 131.95 81.5) (end 131.975 81.525) (width 0.5) (layer "F.Cu") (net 2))
 (segment (start 132.2 81.2) (end 129.2875 84.1125) (width 0.5) (layer "F.Cu") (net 2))
 (segment (start 172.7 88.005679) (end 172.7 81.1) (width 0.5) (layer "F.Cu") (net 2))
 (segment (start 132.25 81.25) (end 132.2 81.2) (width 0.5) (layer "F.Cu") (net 2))
 (segment (start 168.545 106.65) (end 168.545 93.263391) (width 0.5) (layer "F.Cu") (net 2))
 (segment (start 160.445 101.0925) (end 160.445 100.15) (width 0.5) (layer "F.Cu") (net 2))
 (segment (start 158 103.5375) (end 160.445 101.0925) (width 0.5) (layer "F.Cu") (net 2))
 (segment (start 172.7 81.1) (end 148.252144 81.1) (width 0.5) (layer "F.Cu") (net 2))
 (segment (start 142.3 81.25) (end 132.25 81.25) (width 0.5) (layer "F.Cu") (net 2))
 (segment (start 125.15 81.5) (end 131.95 81.5) (width 0.5) (layer "F.Cu") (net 2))
 (segment (start 129.4775 98.9) (end 129.25 98.9) (width 0.5) (layer "F.Cu") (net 2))
 (segment (start 124.5 82.15) (end 125.15 81.5) (width 0.5) (layer "F.Cu") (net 2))
 (segment (start 158.625 104.1625) (end 158 103.5375) (width 0.5) (layer "F.Cu") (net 2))
 (segment (start 158.625 109.1) (end 158.625 104.1625) (width 0.5) (layer "F.Cu") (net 2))
 (segment (start 166.045 109.15) (end 168.545 106.65) (width 0.5) (layer "F.Cu") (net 2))
 (segment (start 158 104.125) (end 158 103.5375) (width 0.5) (layer "F.Cu") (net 2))
 (segment (start 129.4775 98.9) (end 129.4775 105.96) (width 0.5) (layer "F.Cu") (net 2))
 (segment (start 131.75 81.75) (end 131.975 81.525) (width 0.5) (layer "F.Cu") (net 2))
 (segment (start 168.545 93.263391) (end 167.993644 92.712035) (width 0.5) (layer "F.Cu") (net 2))
 (segment (start 163.55 105.574181) (end 163.55 108) (width 0.5) (layer "F.Cu") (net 2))
 (segment (start 131.79474 85.45724) (end 131.75 85.4125) (width 0.5) (layer "F.Cu") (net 2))
 (segment (start 163.55 108) (end 164.7 109.15) (width 0.5) (layer "F.Cu") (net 2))
 (segment (start 124.5 94.15) (end 124.5 82.15) (width 0.5) (layer "F.Cu") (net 2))
 (segment (start 131.75 85.4125) (end 131.75 81.75) (width 0.5) (layer "F.Cu") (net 2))
 (segment (start 135.8 102.95) (end 137.25 104.4) (width 0.5) (layer "F.Cu") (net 10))
 (segment (start 137.25 104.4) (end 137.25 104.95) (width 0.5) (layer "F.Cu") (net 10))
 (segment (start 134.3175 107.8825) (end 137.25 104.95) (width 0.5) (layer "F.Cu") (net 10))
 (segment (start 129.5 107.8825) (end 134.3175 107.8825) (width 0.5) (layer "F.Cu") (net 10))
 (segment (start 139.95 104.95) (end 137.25 104.95) (width 0.5) (layer "F.Cu") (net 10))
 (segment (start 139.95 108.55) (end 141.5 108.55) (width 0.5) (layer "F.Cu") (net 8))
 (segment (start 141.5 108.55) (end 143.3 106.75) (width 0.5) (layer "F.Cu") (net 8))
 (segment (start 159.3 112.2) (end 162.5 112.2) (width 0.5) (layer "F.Cu") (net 7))
 (segment (start 154.8625 101.4625) (end 154.8 101.4) (width 0.5) (layer "F.Cu") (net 3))
 (segment (start 132.529056 94.451) (end 135.8 97.721944) (width 0.5) (layer "F.Cu") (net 3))
 (segment (start 149.305 99.705) (end 149.305 100.695) (width 0.5) (layer "F.Cu") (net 3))
 (segment (start 148 98.4) (end 149.305 99.705) (width 0.5) (layer "F.Cu") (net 3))
 (segment (start 135.8 97.721944) (end 136.478056 98.4) (width 0.5) (layer "F.Cu") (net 3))
 (segment (start 127.2125 85.5) (end 127.2125 92.585) (width 0.5) (layer "F.Cu") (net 3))
 (segment (start 136.478056 98.4) (end 148 98.4) (width 0.5) (layer "F.Cu") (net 3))
 (segment (start 135.8 99.85) (end 135.8 97.721944) (width 0.5) (layer "F.Cu") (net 3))
 (segment (start 154.8 101.4) (end 151.8 98.4) (width 0.5) (layer "F.Cu") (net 3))
 (segment (start 127.1975 92.6) (end 129.0485 94.451) (width 0.5) (layer "F.Cu") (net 3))
 (segment (start 127.2125 92.585) (end 127.1975 92.6) (width 0.5) (layer "F.Cu") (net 3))
 (segment (start 129.0485 94.451) (end 132.529056 94.451) (width 0.5) (layer "F.Cu") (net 3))
 (segment (start 158 101.4625) (end 154.8625 101.4625) (width 0.5) (layer "F.Cu") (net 3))
 (segment (start 151.8 98.4) (end 148 98.4) (width 0.5) (layer "F.Cu") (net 3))
 (segment (start 131.7575 87.495) (end 131.75 87.4875) (width 0.5) (layer "F.Cu") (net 1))
 (segment (start 134.652571 87.4875) (end 131.75 87.4875) (width 0.5) (layer "F.Cu") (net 1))
 (segment (start 136.682831 85.45724) (end 134.652571 87.4875) (width 0.5) (layer "F.Cu") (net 1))
 (segment (start 131.75 92.5925) (end 131.7575 92.6) (width 0.5) (layer "F.Cu") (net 1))
 (segment (start 131.7575 92.6) (end 131.7575 87.495) (width 0.5) (layer "F.Cu") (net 1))
 (segment (start 166.939226 85.460774) (end 162.9 89.5) (width 0.5) (layer "F.Cu") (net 4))
 (segment (start 165.545 103.795) (end 165.545 106.65) (width 0.5) (layer "F.Cu") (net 4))
 (segment (start 167.987267 85.460774) (end 166.939226 85.460774) (width 0.5) (layer "F.Cu") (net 4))
 (segment (start 162.9 101.15) (end 165.545 103.795) (width 0.5) (layer "F.Cu") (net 4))
 (segment (start 162.9 89.5) (end 162.9 101.15) (width 0.5) (layer "F.Cu") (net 4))
 (segment (start 161.545 107.645) (end 161.545 106.65) (width 0.5) (layer "F.Cu") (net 5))
 (segment (start 166.1 112.2) (end 161.545 107.645) (width 0.5) (layer "F.Cu") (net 5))
 (segment (start 166.1 112.2) (end 170.35 112.2) (width 0.5) (layer "F.Cu") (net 5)))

